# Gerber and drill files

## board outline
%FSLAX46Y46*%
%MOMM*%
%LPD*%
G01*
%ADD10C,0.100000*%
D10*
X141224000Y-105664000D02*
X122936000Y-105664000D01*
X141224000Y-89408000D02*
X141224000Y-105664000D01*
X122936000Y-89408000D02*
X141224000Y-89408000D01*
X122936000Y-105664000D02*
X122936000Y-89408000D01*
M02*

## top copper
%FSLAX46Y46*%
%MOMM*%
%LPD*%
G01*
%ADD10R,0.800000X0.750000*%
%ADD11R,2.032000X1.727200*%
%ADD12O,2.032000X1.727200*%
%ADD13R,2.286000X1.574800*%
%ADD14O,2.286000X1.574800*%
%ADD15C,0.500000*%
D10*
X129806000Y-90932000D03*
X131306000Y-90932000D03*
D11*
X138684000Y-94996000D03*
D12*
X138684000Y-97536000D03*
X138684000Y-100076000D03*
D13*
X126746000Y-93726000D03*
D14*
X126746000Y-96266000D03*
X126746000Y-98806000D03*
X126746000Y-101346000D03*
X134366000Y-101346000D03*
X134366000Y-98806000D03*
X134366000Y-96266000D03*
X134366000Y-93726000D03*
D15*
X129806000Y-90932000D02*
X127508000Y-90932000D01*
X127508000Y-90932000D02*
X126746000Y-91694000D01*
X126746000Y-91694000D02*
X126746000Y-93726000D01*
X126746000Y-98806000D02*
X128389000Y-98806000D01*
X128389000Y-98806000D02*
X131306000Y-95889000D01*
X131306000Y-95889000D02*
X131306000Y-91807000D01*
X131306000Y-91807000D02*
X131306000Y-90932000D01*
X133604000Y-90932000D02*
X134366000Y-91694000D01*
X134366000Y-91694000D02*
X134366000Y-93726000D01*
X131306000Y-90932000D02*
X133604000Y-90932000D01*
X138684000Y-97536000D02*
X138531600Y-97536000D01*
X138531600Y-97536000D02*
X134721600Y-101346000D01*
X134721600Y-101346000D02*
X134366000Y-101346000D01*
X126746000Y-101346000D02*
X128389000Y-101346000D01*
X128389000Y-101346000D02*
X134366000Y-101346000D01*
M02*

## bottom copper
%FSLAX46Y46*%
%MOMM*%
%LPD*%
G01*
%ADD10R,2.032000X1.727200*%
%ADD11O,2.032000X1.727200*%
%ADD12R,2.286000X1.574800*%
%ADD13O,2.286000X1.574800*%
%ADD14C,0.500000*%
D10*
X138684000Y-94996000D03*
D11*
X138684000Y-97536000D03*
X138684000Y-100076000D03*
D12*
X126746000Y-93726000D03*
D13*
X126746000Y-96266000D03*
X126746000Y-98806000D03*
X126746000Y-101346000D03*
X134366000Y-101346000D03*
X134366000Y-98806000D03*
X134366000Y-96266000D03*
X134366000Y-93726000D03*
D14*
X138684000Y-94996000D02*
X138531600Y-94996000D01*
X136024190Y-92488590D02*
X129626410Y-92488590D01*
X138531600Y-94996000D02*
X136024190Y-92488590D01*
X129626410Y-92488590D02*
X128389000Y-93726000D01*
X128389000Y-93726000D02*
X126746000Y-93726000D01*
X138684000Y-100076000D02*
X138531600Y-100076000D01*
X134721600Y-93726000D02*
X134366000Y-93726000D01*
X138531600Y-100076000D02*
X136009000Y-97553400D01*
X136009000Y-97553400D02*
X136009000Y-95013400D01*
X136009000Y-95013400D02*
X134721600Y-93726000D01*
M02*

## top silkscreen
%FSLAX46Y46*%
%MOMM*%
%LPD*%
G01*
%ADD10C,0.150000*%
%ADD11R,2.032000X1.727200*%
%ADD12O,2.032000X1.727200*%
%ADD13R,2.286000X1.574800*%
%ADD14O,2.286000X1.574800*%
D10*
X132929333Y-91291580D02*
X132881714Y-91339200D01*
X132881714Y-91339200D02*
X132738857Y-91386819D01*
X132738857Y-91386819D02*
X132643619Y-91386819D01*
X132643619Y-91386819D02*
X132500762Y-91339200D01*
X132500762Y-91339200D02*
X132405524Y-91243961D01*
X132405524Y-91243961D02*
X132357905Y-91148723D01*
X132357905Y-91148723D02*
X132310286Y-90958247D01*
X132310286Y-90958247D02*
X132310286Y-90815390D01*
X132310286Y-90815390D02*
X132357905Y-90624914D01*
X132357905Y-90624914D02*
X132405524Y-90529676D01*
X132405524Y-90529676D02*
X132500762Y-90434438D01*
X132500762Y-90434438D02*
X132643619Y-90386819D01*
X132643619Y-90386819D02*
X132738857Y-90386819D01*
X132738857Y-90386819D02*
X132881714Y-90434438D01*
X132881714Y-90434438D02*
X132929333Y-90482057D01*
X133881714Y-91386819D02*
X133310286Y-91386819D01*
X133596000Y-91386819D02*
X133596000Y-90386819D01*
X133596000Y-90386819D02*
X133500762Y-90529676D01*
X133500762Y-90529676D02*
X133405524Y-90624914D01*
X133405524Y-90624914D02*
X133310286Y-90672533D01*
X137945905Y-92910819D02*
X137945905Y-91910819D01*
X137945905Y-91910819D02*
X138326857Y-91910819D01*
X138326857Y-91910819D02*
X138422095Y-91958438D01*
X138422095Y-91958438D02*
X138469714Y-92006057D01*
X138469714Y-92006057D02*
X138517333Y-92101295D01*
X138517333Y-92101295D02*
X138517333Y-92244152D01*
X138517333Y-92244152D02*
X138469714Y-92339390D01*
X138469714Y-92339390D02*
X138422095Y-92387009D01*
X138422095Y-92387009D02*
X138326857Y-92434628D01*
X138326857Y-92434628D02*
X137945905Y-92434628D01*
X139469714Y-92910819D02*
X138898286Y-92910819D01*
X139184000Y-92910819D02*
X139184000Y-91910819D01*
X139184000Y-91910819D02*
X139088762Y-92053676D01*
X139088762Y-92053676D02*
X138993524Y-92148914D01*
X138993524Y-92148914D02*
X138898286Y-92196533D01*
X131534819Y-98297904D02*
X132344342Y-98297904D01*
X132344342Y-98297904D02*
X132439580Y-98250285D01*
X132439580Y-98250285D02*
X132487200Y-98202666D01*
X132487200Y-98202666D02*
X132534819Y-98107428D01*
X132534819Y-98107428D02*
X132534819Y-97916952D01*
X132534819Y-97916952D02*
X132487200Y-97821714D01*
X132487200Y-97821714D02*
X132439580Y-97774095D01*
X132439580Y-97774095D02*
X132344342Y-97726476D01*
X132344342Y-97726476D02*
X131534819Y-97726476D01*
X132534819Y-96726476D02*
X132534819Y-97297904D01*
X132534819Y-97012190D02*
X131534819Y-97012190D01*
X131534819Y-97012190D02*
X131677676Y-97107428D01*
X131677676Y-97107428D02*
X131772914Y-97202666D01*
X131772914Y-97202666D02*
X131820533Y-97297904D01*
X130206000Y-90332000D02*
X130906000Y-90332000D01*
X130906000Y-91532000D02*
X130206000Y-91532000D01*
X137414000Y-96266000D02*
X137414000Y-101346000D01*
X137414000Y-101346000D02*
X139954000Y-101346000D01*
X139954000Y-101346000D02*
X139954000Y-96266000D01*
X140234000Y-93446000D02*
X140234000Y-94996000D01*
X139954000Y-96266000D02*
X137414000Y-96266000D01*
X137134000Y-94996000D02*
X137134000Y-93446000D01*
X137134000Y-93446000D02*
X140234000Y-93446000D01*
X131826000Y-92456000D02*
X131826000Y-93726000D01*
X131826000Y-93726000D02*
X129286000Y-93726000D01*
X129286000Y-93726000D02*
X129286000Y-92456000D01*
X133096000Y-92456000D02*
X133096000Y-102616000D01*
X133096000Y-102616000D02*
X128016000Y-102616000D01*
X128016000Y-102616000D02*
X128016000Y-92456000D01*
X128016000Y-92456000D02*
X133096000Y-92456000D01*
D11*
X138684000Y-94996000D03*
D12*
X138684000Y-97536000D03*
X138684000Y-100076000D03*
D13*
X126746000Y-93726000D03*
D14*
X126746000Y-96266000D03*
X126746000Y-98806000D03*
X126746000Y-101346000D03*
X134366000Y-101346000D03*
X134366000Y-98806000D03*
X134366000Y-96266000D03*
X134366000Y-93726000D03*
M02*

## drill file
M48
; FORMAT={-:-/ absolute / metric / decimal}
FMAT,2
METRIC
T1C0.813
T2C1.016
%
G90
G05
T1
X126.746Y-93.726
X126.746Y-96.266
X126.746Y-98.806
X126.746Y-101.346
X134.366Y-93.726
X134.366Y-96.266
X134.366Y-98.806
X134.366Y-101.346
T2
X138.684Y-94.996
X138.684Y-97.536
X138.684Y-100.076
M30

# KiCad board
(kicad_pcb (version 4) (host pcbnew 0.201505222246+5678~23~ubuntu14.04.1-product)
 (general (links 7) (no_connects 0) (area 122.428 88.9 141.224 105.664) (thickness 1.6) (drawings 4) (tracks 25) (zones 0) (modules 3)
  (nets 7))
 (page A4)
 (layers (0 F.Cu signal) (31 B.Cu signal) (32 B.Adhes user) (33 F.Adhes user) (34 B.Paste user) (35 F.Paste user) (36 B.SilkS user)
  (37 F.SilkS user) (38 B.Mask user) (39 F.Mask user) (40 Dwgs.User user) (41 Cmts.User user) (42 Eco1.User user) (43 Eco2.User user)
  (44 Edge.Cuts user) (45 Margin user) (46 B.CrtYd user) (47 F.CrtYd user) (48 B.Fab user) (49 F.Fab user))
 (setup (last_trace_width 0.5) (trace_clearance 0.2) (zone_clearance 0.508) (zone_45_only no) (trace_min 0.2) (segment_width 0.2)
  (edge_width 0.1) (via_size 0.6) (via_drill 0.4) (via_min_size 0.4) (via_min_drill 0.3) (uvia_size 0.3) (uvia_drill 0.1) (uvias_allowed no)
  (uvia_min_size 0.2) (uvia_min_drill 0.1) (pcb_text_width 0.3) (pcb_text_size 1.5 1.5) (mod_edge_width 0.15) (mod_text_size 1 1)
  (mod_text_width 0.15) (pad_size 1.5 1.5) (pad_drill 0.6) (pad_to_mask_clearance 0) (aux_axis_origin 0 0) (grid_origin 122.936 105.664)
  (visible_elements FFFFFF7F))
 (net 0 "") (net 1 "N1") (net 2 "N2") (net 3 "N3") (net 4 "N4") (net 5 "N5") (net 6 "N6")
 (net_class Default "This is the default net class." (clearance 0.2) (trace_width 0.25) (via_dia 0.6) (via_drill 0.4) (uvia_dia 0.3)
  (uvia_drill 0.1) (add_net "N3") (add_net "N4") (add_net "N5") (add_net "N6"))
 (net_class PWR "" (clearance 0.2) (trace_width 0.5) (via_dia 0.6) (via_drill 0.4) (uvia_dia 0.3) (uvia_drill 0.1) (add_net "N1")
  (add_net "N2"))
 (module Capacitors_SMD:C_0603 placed (layer F.Cu) (at 130.556 90.932)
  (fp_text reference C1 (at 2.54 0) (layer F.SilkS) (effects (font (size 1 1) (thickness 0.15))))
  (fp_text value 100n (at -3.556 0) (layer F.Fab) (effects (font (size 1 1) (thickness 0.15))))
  (fp_line (start -0.35 -0.6) (end 0.35 -0.6) (layer F.SilkS) (width 0.15))
  (fp_line (start 0.35 0.6) (end -0.35 0.6) (layer F.SilkS) (width 0.15))
  (pad 1 smd rect (at -0.75 0) (size 0.8 0.75) (layers F.Cu F.Paste F.Mask) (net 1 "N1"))
  (pad 2 smd rect (at 0.75 0) (size 0.8 0.75) (layers F.Cu F.Paste F.Mask) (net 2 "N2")))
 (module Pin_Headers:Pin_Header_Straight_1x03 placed (layer F.Cu) (at 138.684 94.996)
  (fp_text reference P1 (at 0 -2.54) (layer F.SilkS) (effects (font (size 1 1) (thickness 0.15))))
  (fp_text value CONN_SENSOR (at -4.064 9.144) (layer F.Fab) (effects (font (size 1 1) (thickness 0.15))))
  (fp_line (start -1.27 1.27) (end -1.27 6.35) (layer F.SilkS) (width 0.15))
  (fp_line (start -1.27 6.35) (end 1.27 6.35) (layer F.SilkS) (width 0.15))
  (fp_line (start 1.27 6.35) (end 1.27 1.27) (layer F.SilkS) (width 0.15))
  (fp_line (start 1.55 -1.55) (end 1.55 0) (layer F.SilkS) (width 0.15))
  (fp_line (start 1.27 1.27) (end -1.27 1.27) (layer F.SilkS) (width 0.15))
  (fp_line (start -1.55 0) (end -1.55 -1.55) (layer F.SilkS) (width 0.15))
  (fp_line (start -1.55 -1.55) (end 1.55 -1.55) (layer F.SilkS) (width 0.15))
  (pad 1 thru_hole rect (at 0 0) (size 2.032 1.7272) (drill 1.016) (layers *.Cu *.Mask F.SilkS) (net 1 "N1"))
  (pad 2 thru_hole oval (at 0 2.54) (size 2.032 1.7272) (drill 1.016) (layers *.Cu *.Mask F.SilkS) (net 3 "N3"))
  (pad 3 thru_hole oval (at 0 5.08) (size 2.032 1.7272) (drill 1.016) (layers *.Cu *.Mask F.SilkS) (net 2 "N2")))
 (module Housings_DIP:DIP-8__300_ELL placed (layer F.Cu) (at 130.556 97.536 270)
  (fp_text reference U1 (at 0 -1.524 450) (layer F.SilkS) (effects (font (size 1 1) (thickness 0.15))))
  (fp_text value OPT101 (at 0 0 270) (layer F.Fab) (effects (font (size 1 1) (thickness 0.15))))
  (fp_line (start -5.08 -1.27) (end -3.81 -1.27) (layer F.SilkS) (width 0.15))
  (fp_line (start -3.81 -1.27) (end -3.81 1.27) (layer F.SilkS) (width 0.15))
  (fp_line (start -3.81 1.27) (end -5.08 1.27) (layer F.SilkS) (width 0.15))
  (fp_line (start -5.08 -2.54) (end 5.08 -2.54) (layer F.SilkS) (width 0.15))
  (fp_line (start 5.08 -2.54) (end 5.08 2.54) (layer F.SilkS) (width 0.15))
  (fp_line (start 5.08 2.54) (end -5.08 2.54) (layer F.SilkS) (width 0.15))
  (fp_line (start -5.08 2.54) (end -5.08 -2.54) (layer F.SilkS) (width 0.15))
  (pad 1 thru_hole rect (at -3.81 3.81 270) (size 1.5748 2.286) (drill 0.8128) (layers *.Cu *.Mask F.SilkS) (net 1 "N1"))
  (pad 2 thru_hole oval (at -1.27 3.81 270) (size 1.5748 2.286) (drill 0.8128) (layers *.Cu *.Mask F.SilkS) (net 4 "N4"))
  (pad 3 thru_hole oval (at 1.27 3.81 270) (size 1.5748 2.286) (drill 0.8128) (layers *.Cu *.Mask F.SilkS) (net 2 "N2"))
  (pad 4 thru_hole oval (at 3.81 3.81 270) (size 1.5748 2.286) (drill 0.8128) (layers *.Cu *.Mask F.SilkS) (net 3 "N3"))
  (pad 5 thru_hole oval (at 3.81 -3.81 270) (size 1.5748 2.286) (drill 0.8128) (layers *.Cu *.Mask F.SilkS) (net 3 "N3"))
  (pad 6 thru_hole oval (at 1.27 -3.81 270) (size 1.5748 2.286) (drill 0.8128) (layers *.Cu *.Mask F.SilkS) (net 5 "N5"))
  (pad 7 thru_hole oval (at -1.27 -3.81 270) (size 1.5748 2.286) (drill 0.8128) (layers *.Cu *.Mask F.SilkS) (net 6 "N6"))
  (pad 8 thru_hole oval (at -3.81 -3.81 270) (size 1.5748 2.286) (drill 0.8128) (layers *.Cu *.Mask F.SilkS) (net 2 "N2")))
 (gr_line (start 141.224 105.664) (end 122.936 105.664) (angle 90) (layer Edge.Cuts) (width 0.1))
 (gr_line (start 141.224 89.408) (end 141.224 105.664) (angle 90) (layer Edge.Cuts) (width 0.1))
 (gr_line (start 122.936 89.408) (end 141.224 89.408) (angle 90) (layer Edge.Cuts) (width 0.1))
 (gr_line (start 122.936 105.664) (end 122.936 89.408) (angle 90) (layer Edge.Cuts) (width 0.1))
 (segment (start 138.684 94.996) (end 138.5316 94.996) (width 0.5) (layer B.Cu) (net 1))
 (segment (start 136.02419 92.48859) (end 129.62641 92.48859) (width 0.5) (layer B.Cu) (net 1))
 (segment (start 138.5316 94.996) (end 136.02419 92.48859) (width 0.5) (layer B.Cu) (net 1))
 (segment (start 129.62641 92.48859) (end 128.389 93.726) (width 0.5) (layer B.Cu) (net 1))
 (segment (start 128.389 93.726) (end 126.746 93.726) (width 0.5) (layer B.Cu) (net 1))
 (segment (start 129.806 90.932) (end 127.508 90.932) (width 0.5) (layer F.Cu) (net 1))
 (segment (start 127.508 90.932) (end 126.746 91.694) (width 0.5) (layer F.Cu) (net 1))
 (segment (start 126.746 91.694) (end 126.746 93.726) (width 0.5) (layer F.Cu) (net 1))
 (segment (start 138.684 100.076) (end 138.5316 100.076) (width 0.5) (layer B.Cu) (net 2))
 (segment (start 134.7216 93.726) (end 134.366 93.726) (width 0.5) (layer B.Cu) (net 2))
 (segment (start 138.5316 100.076) (end 136.009 97.5534) (width 0.5) (layer B.Cu) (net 2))
 (segment (start 136.009 97.5534) (end 136.009 95.0134) (width 0.5) (layer B.Cu) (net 2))
 (segment (start 136.009 95.0134) (end 134.7216 93.726) (width 0.5) (layer B.Cu) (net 2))
 (segment (start 126.746 98.806) (end 128.389 98.806) (width 0.5) (layer F.Cu) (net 2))
 (segment (start 128.389 98.806) (end 131.306 95.889) (width 0.5) (layer F.Cu) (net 2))
 (segment (start 131.306 95.889) (end 131.306 91.807) (width 0.5) (layer F.Cu) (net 2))
 (segment (start 131.306 91.807) (end 131.306 90.932) (width 0.5) (layer F.Cu) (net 2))
 (segment (start 133.604 90.932) (end 134.366 91.694) (width 0.5) (layer F.Cu) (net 2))
 (segment (start 134.366 91.694) (end 134.366 93.726) (width 0.5) (layer F.Cu) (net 2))
 (segment (start 131.306 90.932) (end 133.604 90.932) (width 0.5) (layer F.Cu) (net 2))
 (segment (start 138.684 97.536) (end 138.5316 97.536) (width 0.5) (layer F.Cu) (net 3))
 (segment (start 138.5316 97.536) (end 134.7216 101.346) (width 0.5) (layer F.Cu) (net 3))
 (segment (start 134.7216 101.346) (end 134.366 101.346) (width 0.5) (layer F.Cu) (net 3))
 (segment (start 126.746 101.346) (end 128.389 101.346) (width 0.5) (layer F.Cu) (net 3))
 (segment (start 128.389 101.346) (end 134.366 101.346) (width 0.5) (layer F.Cu) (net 3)))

